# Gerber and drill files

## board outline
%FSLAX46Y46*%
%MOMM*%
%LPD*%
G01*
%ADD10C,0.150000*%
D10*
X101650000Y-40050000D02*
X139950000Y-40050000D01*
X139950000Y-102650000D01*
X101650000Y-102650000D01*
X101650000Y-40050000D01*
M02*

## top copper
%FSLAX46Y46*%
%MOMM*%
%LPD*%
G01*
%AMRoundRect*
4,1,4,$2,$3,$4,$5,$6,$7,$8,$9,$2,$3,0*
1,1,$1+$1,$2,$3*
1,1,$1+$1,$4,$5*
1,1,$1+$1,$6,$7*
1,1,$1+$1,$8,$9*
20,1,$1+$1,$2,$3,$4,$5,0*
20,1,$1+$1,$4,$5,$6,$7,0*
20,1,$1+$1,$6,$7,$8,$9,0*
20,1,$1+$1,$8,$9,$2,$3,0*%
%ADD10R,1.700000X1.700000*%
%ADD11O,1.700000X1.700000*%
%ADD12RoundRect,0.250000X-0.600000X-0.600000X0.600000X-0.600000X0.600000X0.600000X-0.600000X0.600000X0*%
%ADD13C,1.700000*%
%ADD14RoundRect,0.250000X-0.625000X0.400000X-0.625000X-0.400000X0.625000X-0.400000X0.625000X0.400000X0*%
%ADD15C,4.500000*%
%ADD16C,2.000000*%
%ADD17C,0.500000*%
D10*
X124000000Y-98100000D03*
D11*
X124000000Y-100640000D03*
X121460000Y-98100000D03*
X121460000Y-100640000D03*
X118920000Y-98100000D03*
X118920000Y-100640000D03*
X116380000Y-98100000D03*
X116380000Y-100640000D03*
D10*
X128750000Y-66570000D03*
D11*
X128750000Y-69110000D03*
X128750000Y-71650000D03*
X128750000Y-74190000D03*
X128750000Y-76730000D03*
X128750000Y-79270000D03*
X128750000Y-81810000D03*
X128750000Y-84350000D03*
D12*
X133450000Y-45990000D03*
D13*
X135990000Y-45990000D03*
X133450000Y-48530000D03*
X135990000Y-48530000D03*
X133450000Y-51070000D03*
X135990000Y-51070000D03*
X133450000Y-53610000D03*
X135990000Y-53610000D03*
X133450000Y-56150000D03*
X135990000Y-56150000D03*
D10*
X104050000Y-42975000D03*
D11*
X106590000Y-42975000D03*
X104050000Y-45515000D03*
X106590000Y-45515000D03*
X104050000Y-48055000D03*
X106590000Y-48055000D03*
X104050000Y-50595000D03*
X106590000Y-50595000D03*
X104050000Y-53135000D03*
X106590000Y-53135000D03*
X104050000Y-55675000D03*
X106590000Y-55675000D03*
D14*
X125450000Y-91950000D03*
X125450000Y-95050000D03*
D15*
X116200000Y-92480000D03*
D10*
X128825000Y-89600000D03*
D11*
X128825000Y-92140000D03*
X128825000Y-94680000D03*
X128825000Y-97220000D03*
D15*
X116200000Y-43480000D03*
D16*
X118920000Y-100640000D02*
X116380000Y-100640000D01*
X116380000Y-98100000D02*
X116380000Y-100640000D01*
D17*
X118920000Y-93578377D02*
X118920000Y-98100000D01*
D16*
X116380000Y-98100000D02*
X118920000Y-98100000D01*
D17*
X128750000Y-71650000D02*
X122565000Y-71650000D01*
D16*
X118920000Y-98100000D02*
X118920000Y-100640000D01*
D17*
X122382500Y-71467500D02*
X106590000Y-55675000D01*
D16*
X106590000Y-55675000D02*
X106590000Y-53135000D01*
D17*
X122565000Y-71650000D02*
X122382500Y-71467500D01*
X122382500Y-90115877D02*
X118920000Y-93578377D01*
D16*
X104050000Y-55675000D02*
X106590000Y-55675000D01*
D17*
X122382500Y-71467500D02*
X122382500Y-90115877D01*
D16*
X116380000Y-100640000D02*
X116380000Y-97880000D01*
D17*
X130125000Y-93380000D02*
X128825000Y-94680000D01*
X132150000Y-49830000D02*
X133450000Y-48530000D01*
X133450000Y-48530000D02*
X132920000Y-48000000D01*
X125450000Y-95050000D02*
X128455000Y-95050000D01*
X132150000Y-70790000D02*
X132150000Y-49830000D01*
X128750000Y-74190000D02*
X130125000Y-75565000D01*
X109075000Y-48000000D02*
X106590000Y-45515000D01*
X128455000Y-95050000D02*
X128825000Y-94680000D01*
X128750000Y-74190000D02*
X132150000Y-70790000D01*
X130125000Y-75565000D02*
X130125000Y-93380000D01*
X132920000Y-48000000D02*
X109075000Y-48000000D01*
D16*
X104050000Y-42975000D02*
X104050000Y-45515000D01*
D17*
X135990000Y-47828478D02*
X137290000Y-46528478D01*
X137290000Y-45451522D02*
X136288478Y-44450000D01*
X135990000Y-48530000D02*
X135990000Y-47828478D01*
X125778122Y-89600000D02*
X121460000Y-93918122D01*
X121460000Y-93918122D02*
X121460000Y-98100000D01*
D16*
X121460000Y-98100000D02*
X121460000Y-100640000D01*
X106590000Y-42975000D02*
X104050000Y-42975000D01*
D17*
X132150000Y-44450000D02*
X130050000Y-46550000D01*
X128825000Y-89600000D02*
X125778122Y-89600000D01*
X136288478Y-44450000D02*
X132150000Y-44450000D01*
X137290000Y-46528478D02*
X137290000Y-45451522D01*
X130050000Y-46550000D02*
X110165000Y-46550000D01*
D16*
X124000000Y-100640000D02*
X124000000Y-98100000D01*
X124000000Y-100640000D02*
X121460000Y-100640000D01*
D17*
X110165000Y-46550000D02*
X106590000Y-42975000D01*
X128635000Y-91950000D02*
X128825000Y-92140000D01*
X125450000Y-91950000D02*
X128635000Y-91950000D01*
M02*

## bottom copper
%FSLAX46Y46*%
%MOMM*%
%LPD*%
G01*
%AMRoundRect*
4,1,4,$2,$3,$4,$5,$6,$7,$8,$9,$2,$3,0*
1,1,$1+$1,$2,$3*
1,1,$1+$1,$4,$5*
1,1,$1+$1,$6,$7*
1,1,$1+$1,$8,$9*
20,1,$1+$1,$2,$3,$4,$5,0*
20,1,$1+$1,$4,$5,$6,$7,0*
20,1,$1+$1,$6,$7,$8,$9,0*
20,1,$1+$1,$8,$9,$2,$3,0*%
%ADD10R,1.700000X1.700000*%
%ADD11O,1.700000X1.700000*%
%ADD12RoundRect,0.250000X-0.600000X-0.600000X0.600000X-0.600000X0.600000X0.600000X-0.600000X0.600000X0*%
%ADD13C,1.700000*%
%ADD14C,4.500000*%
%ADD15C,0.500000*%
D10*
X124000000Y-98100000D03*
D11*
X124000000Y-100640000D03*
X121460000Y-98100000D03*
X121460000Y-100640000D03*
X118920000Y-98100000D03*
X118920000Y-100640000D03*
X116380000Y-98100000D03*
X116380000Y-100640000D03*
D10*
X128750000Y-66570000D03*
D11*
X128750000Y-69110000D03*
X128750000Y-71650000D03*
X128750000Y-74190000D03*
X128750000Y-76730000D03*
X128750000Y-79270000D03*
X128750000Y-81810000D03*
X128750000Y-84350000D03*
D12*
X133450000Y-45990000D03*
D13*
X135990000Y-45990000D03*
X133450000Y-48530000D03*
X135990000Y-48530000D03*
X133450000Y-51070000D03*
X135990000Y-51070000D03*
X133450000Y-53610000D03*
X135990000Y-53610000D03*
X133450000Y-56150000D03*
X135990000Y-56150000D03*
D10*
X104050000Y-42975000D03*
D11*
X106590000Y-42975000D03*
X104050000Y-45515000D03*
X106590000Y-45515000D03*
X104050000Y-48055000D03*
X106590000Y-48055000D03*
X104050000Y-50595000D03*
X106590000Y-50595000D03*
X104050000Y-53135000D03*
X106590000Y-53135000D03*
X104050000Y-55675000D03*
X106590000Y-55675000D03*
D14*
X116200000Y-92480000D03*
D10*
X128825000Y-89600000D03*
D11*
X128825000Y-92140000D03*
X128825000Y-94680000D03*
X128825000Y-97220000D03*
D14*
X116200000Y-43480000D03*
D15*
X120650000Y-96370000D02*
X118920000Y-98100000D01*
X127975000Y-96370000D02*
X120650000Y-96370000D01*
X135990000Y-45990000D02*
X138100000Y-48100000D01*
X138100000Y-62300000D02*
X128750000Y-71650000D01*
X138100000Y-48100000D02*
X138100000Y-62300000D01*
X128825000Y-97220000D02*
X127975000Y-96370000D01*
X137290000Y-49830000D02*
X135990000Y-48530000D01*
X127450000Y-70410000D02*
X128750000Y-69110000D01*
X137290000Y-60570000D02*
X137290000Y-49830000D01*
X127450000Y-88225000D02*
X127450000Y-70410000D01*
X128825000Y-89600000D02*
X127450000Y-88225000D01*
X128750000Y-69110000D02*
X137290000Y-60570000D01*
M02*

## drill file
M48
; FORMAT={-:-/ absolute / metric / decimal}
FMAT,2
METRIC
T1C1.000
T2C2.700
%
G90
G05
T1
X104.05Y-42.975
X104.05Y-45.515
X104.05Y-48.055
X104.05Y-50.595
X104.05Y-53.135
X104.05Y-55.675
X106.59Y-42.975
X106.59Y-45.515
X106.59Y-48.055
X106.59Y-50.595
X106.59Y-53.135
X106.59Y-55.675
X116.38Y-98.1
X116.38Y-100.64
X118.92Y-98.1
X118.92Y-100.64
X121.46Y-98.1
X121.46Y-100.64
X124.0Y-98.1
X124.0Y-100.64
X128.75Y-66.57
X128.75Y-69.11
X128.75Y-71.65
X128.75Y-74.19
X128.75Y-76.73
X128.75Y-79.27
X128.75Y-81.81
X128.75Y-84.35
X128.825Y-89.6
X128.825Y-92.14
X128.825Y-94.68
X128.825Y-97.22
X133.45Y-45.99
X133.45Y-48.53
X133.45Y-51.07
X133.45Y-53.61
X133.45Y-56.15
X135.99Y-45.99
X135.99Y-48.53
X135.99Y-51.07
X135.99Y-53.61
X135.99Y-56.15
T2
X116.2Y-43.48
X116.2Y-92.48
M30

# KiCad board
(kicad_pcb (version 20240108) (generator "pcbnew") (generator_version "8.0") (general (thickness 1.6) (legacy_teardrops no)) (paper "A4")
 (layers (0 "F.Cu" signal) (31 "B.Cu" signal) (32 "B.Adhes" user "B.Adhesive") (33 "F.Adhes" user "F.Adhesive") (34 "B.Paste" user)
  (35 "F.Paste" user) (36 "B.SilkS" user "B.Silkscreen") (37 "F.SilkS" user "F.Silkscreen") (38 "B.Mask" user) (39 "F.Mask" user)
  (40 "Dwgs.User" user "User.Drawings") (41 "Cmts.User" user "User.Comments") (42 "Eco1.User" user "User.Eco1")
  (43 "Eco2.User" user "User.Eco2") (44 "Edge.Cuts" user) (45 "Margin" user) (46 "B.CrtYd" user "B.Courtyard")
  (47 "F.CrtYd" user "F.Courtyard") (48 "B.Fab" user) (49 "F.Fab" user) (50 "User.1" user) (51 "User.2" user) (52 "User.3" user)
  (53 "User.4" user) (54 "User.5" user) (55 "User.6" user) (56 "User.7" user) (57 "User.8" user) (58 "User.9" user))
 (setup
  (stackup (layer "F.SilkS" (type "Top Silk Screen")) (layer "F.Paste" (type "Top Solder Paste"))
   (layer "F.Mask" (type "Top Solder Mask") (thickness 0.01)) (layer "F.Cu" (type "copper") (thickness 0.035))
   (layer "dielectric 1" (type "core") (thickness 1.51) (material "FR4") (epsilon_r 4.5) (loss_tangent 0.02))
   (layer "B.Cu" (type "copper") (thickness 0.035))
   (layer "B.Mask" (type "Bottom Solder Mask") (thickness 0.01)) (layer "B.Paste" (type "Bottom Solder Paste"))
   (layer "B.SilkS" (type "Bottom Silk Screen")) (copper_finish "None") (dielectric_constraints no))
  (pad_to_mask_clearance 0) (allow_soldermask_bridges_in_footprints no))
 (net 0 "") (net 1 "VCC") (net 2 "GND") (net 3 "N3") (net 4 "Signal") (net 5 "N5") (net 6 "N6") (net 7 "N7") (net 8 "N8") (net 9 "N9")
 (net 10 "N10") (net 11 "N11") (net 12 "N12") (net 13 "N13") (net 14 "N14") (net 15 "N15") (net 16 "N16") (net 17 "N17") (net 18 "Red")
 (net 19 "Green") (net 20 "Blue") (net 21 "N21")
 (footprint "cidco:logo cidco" (layer "F.Cu") (at 113.75 73.78)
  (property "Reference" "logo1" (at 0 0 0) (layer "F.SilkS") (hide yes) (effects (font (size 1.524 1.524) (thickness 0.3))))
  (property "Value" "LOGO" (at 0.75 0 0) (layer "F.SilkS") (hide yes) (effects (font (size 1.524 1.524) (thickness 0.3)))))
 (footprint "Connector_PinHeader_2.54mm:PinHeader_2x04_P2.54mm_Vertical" (layer "F.Cu") (at 124 98.1 -90)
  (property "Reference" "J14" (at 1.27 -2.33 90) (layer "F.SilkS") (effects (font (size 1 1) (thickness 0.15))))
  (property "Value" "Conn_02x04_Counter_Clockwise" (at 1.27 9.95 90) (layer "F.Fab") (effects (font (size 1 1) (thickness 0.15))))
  (pad "1" thru_hole rect (at 0 0 270) (size 1.7 1.7) (drill 1) (layers "*.Cu" "*.Mask") (remove_unused_layers no) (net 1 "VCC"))
  (pad "2" thru_hole oval (at 2.54 0 270) (size 1.7 1.7) (drill 1) (layers "*.Cu" "*.Mask") (remove_unused_layers no) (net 1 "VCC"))
  (pad "3" thru_hole oval (at 0 2.54 270) (size 1.7 1.7) (drill 1) (layers "*.Cu" "*.Mask") (remove_unused_layers no) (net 1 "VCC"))
  (pad "4" thru_hole oval (at 2.54 2.54 270) (size 1.7 1.7) (drill 1) (layers "*.Cu" "*.Mask") (remove_unused_layers no) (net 1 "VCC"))
  (pad "5" thru_hole oval (at 0 5.08 270) (size 1.7 1.7) (drill 1) (layers "*.Cu" "*.Mask") (remove_unused_layers no) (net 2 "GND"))
  (pad "6" thru_hole oval (at 2.54 5.08 270) (size 1.7 1.7) (drill 1) (layers "*.Cu" "*.Mask") (remove_unused_layers no) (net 2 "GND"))
  (pad "7" thru_hole oval (at 0 7.62 270) (size 1.7 1.7) (drill 1) (layers "*.Cu" "*.Mask") (remove_unused_layers no) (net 2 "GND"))
  (pad "8" thru_hole oval (at 2.54 7.62 270) (size 1.7 1.7) (drill 1) (layers "*.Cu" "*.Mask") (remove_unused_layers no) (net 2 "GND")))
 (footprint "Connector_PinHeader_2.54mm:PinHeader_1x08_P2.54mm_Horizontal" (layer "F.Cu") (at 128.75 66.57)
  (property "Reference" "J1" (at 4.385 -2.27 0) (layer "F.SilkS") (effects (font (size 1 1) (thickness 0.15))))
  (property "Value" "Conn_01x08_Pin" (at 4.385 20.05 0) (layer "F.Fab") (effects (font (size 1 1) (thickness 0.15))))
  (pad "1" thru_hole rect (at 0 0) (size 1.7 1.7) (drill 1) (layers "*.Cu" "*.Mask") (remove_unused_layers no) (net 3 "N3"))
  (pad "2" thru_hole oval (at 0 2.54) (size 1.7 1.7) (drill 1) (layers "*.Cu" "*.Mask") (remove_unused_layers no) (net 1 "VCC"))
  (pad "3" thru_hole oval (at 0 5.08) (size 1.7 1.7) (drill 1) (layers "*.Cu" "*.Mask") (remove_unused_layers no) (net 2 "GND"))
  (pad "4" thru_hole oval (at 0 7.62) (size 1.7 1.7) (drill 1) (layers "*.Cu" "*.Mask") (remove_unused_layers no) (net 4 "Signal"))
  (pad "5" thru_hole oval (at 0 10.16) (size 1.7 1.7) (drill 1) (layers "*.Cu" "*.Mask") (remove_unused_layers no) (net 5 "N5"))
  (pad "6" thru_hole oval (at 0 12.7) (size 1.7 1.7) (drill 1) (layers "*.Cu" "*.Mask") (remove_unused_layers no) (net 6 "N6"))
  (pad "7" thru_hole oval (at 0 15.24) (size 1.7 1.7) (drill 1) (layers "*.Cu" "*.Mask") (remove_unused_layers no) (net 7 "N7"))
  (pad "8" thru_hole oval (at 0 17.78) (size 1.7 1.7) (drill 1) (layers "*.Cu" "*.Mask") (remove_unused_layers no) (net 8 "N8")))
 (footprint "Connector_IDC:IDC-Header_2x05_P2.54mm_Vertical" (layer "F.Cu") (at 133.45 45.99)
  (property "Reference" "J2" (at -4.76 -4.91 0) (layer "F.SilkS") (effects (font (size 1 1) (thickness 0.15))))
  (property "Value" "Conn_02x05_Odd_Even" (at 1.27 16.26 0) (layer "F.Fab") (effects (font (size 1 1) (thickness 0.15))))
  (pad "1" thru_hole roundrect (at 0 0) (size 1.7 1.7) (drill 1) (layers "*.Cu" "*.Mask") (remove_unused_layers no)
   (roundrect_rratio 0.147059) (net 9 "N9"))
  (pad "2" thru_hole circle (at 2.54 0) (size 1.7 1.7) (drill 1) (layers "*.Cu" "*.Mask") (remove_unused_layers no) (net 2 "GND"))
  (pad "3" thru_hole circle (at 0 2.54) (size 1.7 1.7) (drill 1) (layers "*.Cu" "*.Mask") (remove_unused_layers no) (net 4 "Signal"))
  (pad "4" thru_hole circle (at 2.54 2.54) (size 1.7 1.7) (drill 1) (layers "*.Cu" "*.Mask") (remove_unused_layers no) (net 1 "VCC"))
  (pad "5" thru_hole circle (at 0 5.08) (size 1.7 1.7) (drill 1) (layers "*.Cu" "*.Mask") (remove_unused_layers no) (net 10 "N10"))
  (pad "6" thru_hole circle (at 2.54 5.08) (size 1.7 1.7) (drill 1) (layers "*.Cu" "*.Mask") (remove_unused_layers no) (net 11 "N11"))
  (pad "7" thru_hole circle (at 0 7.62) (size 1.7 1.7) (drill 1) (layers "*.Cu" "*.Mask") (remove_unused_layers no) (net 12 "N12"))
  (pad "8" thru_hole circle (at 2.54 7.62) (size 1.7 1.7) (drill 1) (layers "*.Cu" "*.Mask") (remove_unused_layers no) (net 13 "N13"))
  (pad "9" thru_hole circle (at 0 10.16) (size 1.7 1.7) (drill 1) (layers "*.Cu" "*.Mask") (remove_unused_layers no) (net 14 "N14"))
  (pad "10" thru_hole circle (at 2.54 10.16) (size 1.7 1.7) (drill 1) (layers "*.Cu" "*.Mask") (remove_unused_layers no) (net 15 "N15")))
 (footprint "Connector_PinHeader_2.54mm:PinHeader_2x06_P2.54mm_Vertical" (layer "F.Cu") (at 104.05 42.975)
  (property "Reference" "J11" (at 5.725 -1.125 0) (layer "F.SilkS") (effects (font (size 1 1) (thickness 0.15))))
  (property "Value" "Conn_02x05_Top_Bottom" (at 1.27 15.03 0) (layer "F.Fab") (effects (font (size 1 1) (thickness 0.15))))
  (pad "1" thru_hole rect (at 0 0) (size 1.7 1.7) (drill 1) (layers "*.Cu" "*.Mask") (remove_unused_layers no) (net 1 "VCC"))
  (pad "2" thru_hole oval (at 2.54 0) (size 1.7 1.7) (drill 1) (layers "*.Cu" "*.Mask") (remove_unused_layers no) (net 1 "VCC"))
  (pad "3" thru_hole oval (at 0 2.54) (size 1.7 1.7) (drill 1) (layers "*.Cu" "*.Mask") (remove_unused_layers no) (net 1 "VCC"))
  (pad "4" thru_hole oval (at 2.54 2.54) (size 1.7 1.7) (drill 1) (layers "*.Cu" "*.Mask") (remove_unused_layers no) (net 4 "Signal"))
  (pad "5" thru_hole oval (at 0 5.08) (size 1.7 1.7) (drill 1) (layers "*.Cu" "*.Mask") (remove_unused_layers no) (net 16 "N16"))
  (pad "6" thru_hole oval (at 2.54 5.08) (size 1.7 1.7) (drill 1) (layers "*.Cu" "*.Mask") (remove_unused_layers no) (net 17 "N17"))
  (pad "7" thru_hole oval (at 0 7.62) (size 1.7 1.7) (drill 1) (layers "*.Cu" "*.Mask") (remove_unused_layers no) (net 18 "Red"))
  (pad "8" thru_hole oval (at 2.54 7.62) (size 1.7 1.7) (drill 1) (layers "*.Cu" "*.Mask") (remove_unused_layers no) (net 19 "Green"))
  (pad "9" thru_hole oval (at 0 10.16) (size 1.7 1.7) (drill 1) (layers "*.Cu" "*.Mask") (remove_unused_layers no) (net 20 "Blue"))
  (pad "10" thru_hole oval (at 2.54 10.16) (size 1.7 1.7) (drill 1) (layers "*.Cu" "*.Mask") (remove_unused_layers no) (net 2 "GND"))
  (pad "11" thru_hole oval (at 0 12.7) (size 1.7 1.7) (drill 1) (layers "*.Cu" "*.Mask") (remove_unused_layers no) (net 2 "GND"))
  (pad "12" thru_hole oval (at 2.54 12.7) (size 1.7 1.7) (drill 1) (layers "*.Cu" "*.Mask") (remove_unused_layers no) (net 2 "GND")))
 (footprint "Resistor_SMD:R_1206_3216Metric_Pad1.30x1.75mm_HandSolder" (layer "F.Cu") (at 125.45 93.5 -90)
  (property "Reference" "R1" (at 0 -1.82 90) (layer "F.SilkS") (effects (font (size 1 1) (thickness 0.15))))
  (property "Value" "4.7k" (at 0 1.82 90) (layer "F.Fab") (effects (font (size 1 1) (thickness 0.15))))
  (pad "1" smd roundrect (at -1.55 0 270) (size 1.3 1.75) (layers "F.Cu" "F.Paste" "F.Mask") (roundrect_rratio 0.192308) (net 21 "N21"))
  (pad "2" smd roundrect (at 1.55 0 270) (size 1.3 1.75) (layers "F.Cu" "F.Paste" "F.Mask") (roundrect_rratio 0.192308) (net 4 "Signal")))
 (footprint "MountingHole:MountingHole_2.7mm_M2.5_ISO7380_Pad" (layer "F.Cu") (at 116.2 92.48)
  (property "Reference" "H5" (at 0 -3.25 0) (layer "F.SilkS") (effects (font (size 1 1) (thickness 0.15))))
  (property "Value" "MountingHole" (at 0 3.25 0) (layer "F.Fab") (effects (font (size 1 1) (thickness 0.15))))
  (pad "1" thru_hole circle (at 0 0) (size 4.5 4.5) (drill 2.7) (layers "*.Cu" "*.Mask") (remove_unused_layers no)))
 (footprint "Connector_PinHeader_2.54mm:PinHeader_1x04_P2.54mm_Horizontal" (layer "F.Cu") (at 128.825 89.6)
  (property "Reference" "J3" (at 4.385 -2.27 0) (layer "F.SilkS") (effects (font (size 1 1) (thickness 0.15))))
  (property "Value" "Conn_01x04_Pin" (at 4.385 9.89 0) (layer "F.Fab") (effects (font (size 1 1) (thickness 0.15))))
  (pad "1" thru_hole rect (at 0 0) (size 1.7 1.7) (drill 1) (layers "*.Cu" "*.Mask") (remove_unused_layers no) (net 1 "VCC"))
  (pad "2" thru_hole oval (at 0 2.54) (size 1.7 1.7) (drill 1) (layers "*.Cu" "*.Mask") (remove_unused_layers no) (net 21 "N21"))
  (pad "3" thru_hole oval (at 0 5.08) (size 1.7 1.7) (drill 1) (layers "*.Cu" "*.Mask") (remove_unused_layers no) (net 4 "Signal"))
  (pad "4" thru_hole oval (at 0 7.62) (size 1.7 1.7) (drill 1) (layers "*.Cu" "*.Mask") (remove_unused_layers no) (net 2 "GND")))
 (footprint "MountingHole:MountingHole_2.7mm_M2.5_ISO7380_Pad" (layer "F.Cu") (at 116.2 43.48)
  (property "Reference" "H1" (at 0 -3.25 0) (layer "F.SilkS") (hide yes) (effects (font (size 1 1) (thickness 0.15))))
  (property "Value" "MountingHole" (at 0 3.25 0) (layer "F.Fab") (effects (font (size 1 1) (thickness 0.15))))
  (pad "1" thru_hole circle (at 0 0) (size 4.5 4.5) (drill 2.7) (layers "*.Cu" "*.Mask") (remove_unused_layers no)))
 (gr_rect (start 101.65 40.05) (end 139.95 102.65) (stroke (width 0.15) (type default)) (fill none) (layer "Edge.Cuts"))
 (segment (start 118.92 100.64) (end 116.38 100.64) (width 2) (layer "F.Cu") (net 2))
 (segment (start 116.38 98.1) (end 116.38 100.64) (width 2) (layer "F.Cu") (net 2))
 (segment (start 118.92 93.578377) (end 118.92 98.1) (width 0.5) (layer "F.Cu") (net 2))
 (segment (start 116.38 98.1) (end 118.92 98.1) (width 2) (layer "F.Cu") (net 2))
 (segment (start 128.75 71.65) (end 122.565 71.65) (width 0.5) (layer "F.Cu") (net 2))
 (segment (start 118.92 98.1) (end 118.92 100.64) (width 2) (layer "F.Cu") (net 2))
 (segment (start 122.3825 71.4675) (end 106.59 55.675) (width 0.5) (layer "F.Cu") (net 2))
 (segment (start 106.59 55.675) (end 106.59 53.135) (width 2) (layer "F.Cu") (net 2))
 (segment (start 122.565 71.65) (end 122.3825 71.4675) (width 0.5) (layer "F.Cu") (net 2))
 (segment (start 122.3825 90.115877) (end 118.92 93.578377) (width 0.5) (layer "F.Cu") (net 2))
 (segment (start 104.05 55.675) (end 106.59 55.675) (width 2) (layer "F.Cu") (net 2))
 (segment (start 122.3825 71.4675) (end 122.3825 90.115877) (width 0.5) (layer "F.Cu") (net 2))
 (segment (start 116.38 100.64) (end 116.38 97.88) (width 2) (layer "F.Cu") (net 2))
 (segment (start 120.65 96.37) (end 118.92 98.1) (width 0.5) (layer "B.Cu") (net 2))
 (segment (start 127.975 96.37) (end 120.65 96.37) (width 0.5) (layer "B.Cu") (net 2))
 (segment (start 135.99 45.99) (end 138.1 48.1) (width 0.5) (layer "B.Cu") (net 2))
 (segment (start 138.1 62.3) (end 128.75 71.65) (width 0.5) (layer "B.Cu") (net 2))
 (segment (start 138.1 48.1) (end 138.1 62.3) (width 0.5) (layer "B.Cu") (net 2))
 (segment (start 128.825 97.22) (end 127.975 96.37) (width 0.5) (layer "B.Cu") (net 2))
 (segment (start 130.125 93.38) (end 128.825 94.68) (width 0.5) (layer "F.Cu") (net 4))
 (segment (start 132.15 49.83) (end 133.45 48.53) (width 0.5) (layer "F.Cu") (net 4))
 (segment (start 133.45 48.53) (end 132.92 48) (width 0.5) (layer "F.Cu") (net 4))
 (segment (start 125.45 95.05) (end 128.455 95.05) (width 0.5) (layer "F.Cu") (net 4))
 (segment (start 132.15 70.79) (end 132.15 49.83) (width 0.5) (layer "F.Cu") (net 4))
 (segment (start 128.75 74.19) (end 130.125 75.565) (width 0.5) (layer "F.Cu") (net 4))
 (segment (start 109.075 48) (end 106.59 45.515) (width 0.5) (layer "F.Cu") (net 4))
 (segment (start 128.455 95.05) (end 128.825 94.68) (width 0.5) (layer "F.Cu") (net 4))
 (segment (start 128.75 74.19) (end 132.15 70.79) (width 0.5) (layer "F.Cu") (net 4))
 (segment (start 130.125 75.565) (end 130.125 93.38) (width 0.5) (layer "F.Cu") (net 4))
 (segment (start 132.92 48) (end 109.075 48) (width 0.5) (layer "F.Cu") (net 4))
 (segment (start 104.05 42.975) (end 104.05 45.515) (width 2) (layer "F.Cu") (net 1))
 (segment (start 135.99 47.828478) (end 137.29 46.528478) (width 0.5) (layer "F.Cu") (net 1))
 (segment (start 137.29 45.451522) (end 136.288478 44.45) (width 0.5) (layer "F.Cu") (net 1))
 (segment (start 135.99 48.53) (end 135.99 47.828478) (width 0.5) (layer "F.Cu") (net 1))
 (segment (start 125.778122 89.6) (end 121.46 93.918122) (width 0.5) (layer "F.Cu") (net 1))
 (segment (start 121.46 93.918122) (end 121.46 98.1) (width 0.5) (layer "F.Cu") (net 1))
 (segment (start 121.46 98.1) (end 121.46 100.64) (width 2) (layer "F.Cu") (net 1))
 (segment (start 106.59 42.975) (end 104.05 42.975) (width 2) (layer "F.Cu") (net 1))
 (segment (start 132.15 44.45) (end 130.05 46.55) (width 0.5) (layer "F.Cu") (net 1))
 (segment (start 128.825 89.6) (end 125.778122 89.6) (width 0.5) (layer "F.Cu") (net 1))
 (segment (start 136.288478 44.45) (end 132.15 44.45) (width 0.5) (layer "F.Cu") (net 1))
 (segment (start 137.29 46.528478) (end 137.29 45.451522) (width 0.5) (layer "F.Cu") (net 1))
 (segment (start 130.05 46.55) (end 110.165 46.55) (width 0.5) (layer "F.Cu") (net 1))
 (segment (start 124 100.64) (end 124 98.1) (width 2) (layer "F.Cu") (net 1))
 (segment (start 124 100.64) (end 121.46 100.64) (width 2) (layer "F.Cu") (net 1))
 (segment (start 110.165 46.55) (end 106.59 42.975) (width 0.5) (layer "F.Cu") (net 1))
 (segment (start 137.29 49.83) (end 135.99 48.53) (width 0.5) (layer "B.Cu") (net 1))
 (segment (start 127.45 70.41) (end 128.75 69.11) (width 0.5) (layer "B.Cu") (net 1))
 (segment (start 137.29 60.57) (end 137.29 49.83) (width 0.5) (layer "B.Cu") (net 1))
 (segment (start 127.45 88.225) (end 127.45 70.41) (width 0.5) (layer "B.Cu") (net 1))
 (segment (start 128.825 89.6) (end 127.45 88.225) (width 0.5) (layer "B.Cu") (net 1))
 (segment (start 128.75 69.11) (end 137.29 60.57) (width 0.5) (layer "B.Cu") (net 1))
 (segment (start 128.635 91.95) (end 128.825 92.14) (width 0.5) (layer "F.Cu") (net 21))
 (segment (start 125.45 91.95) (end 128.635 91.95) (width 0.5) (layer "F.Cu") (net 21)))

